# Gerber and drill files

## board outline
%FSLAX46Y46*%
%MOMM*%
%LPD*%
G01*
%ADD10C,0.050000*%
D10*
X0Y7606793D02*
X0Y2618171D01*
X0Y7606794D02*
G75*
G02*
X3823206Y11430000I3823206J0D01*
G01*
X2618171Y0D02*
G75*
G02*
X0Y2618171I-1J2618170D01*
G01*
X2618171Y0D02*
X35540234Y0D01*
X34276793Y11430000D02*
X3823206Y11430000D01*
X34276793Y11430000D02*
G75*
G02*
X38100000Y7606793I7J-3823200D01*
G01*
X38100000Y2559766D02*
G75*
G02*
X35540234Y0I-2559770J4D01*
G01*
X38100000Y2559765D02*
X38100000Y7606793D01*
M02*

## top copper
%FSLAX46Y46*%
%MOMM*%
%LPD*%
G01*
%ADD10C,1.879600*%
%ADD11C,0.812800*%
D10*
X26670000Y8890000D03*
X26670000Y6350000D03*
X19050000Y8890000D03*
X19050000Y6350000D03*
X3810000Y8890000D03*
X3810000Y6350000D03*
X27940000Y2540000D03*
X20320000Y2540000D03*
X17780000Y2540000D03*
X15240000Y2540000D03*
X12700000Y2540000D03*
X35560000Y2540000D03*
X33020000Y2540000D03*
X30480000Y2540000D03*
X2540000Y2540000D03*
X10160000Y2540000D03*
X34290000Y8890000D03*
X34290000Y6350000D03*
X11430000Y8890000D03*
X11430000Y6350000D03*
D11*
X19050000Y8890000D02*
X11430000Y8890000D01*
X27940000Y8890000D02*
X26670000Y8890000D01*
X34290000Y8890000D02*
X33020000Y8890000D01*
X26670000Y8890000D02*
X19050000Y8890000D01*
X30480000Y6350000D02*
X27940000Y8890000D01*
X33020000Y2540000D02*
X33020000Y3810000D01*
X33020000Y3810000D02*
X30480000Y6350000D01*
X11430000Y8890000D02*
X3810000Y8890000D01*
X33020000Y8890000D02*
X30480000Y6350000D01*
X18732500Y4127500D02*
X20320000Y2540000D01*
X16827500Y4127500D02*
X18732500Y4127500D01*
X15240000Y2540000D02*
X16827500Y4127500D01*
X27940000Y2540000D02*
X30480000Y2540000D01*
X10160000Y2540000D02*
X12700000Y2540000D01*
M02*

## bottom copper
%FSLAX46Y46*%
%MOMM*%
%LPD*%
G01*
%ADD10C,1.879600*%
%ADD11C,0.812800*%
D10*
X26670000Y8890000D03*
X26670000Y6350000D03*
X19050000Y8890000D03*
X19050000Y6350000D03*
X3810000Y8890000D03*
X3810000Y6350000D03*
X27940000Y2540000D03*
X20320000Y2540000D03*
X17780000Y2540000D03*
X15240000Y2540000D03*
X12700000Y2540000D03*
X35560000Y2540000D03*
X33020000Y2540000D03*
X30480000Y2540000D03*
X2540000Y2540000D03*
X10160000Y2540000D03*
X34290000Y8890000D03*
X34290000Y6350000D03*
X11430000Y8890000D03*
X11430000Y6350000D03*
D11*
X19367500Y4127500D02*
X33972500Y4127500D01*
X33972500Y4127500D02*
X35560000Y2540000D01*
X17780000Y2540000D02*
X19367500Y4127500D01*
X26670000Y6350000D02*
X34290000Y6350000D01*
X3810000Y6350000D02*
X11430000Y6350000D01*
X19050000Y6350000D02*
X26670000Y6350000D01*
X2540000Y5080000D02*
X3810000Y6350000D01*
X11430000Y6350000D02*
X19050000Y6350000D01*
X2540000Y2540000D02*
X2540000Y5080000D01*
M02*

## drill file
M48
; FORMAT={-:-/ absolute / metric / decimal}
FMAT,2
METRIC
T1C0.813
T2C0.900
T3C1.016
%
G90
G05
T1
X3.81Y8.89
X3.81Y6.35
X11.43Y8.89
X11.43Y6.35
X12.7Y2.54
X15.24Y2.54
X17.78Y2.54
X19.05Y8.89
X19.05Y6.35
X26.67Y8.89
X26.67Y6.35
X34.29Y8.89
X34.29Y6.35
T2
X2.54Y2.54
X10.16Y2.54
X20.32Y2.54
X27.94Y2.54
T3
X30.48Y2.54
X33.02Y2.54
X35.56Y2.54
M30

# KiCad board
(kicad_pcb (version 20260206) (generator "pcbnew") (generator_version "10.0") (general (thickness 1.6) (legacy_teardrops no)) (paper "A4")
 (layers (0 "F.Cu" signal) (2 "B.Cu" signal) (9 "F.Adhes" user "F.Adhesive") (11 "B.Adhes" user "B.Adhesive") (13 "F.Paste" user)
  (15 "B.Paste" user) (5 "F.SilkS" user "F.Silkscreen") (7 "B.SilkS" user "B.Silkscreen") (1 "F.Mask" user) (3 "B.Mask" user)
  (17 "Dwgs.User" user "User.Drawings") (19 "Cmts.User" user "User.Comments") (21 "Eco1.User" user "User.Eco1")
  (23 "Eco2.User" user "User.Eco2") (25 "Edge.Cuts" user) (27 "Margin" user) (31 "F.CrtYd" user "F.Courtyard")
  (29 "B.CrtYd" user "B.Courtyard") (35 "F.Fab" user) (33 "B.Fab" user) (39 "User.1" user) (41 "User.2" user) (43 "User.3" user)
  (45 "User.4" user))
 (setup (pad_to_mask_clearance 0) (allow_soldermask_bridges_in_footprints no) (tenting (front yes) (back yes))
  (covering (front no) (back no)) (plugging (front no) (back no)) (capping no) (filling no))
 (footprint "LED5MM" (layer "F.Cu") (at 26.67 -7.62 -90)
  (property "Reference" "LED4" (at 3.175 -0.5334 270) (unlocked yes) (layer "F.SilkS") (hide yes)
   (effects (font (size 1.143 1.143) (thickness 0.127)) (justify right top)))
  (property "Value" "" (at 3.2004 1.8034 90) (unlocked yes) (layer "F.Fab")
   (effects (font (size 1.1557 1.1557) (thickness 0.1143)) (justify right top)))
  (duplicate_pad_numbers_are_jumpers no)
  (pad "A" thru_hole circle (at -1.27 0 270) (size 1.8796 1.8796) (drill 0.8128) (layers "*.Cu" "*.Mask") (remove_unused_layers no)
   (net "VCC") (solder_mask_margin 0.1016) (thermal_bridge_angle 0))
  (pad "K" thru_hole circle (at 1.27 0 270) (size 1.8796 1.8796) (drill 0.8128) (layers "*.Cu" "*.Mask") (remove_unused_layers no)
   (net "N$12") (solder_mask_margin 0.1016) (thermal_bridge_angle 0)))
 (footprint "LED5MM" (layer "F.Cu") (at 19.05 -7.62 -90)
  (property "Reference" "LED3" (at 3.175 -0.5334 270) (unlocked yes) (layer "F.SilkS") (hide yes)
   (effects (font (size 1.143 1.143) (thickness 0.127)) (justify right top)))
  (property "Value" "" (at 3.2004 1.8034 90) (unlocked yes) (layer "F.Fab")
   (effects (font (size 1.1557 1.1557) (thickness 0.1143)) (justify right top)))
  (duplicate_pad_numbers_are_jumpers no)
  (pad "A" thru_hole circle (at -1.27 0 270) (size 1.8796 1.8796) (drill 0.8128) (layers "*.Cu" "*.Mask") (remove_unused_layers no)
   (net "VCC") (solder_mask_margin 0.1016) (thermal_bridge_angle 0))
  (pad "K" thru_hole circle (at 1.27 0 270) (size 1.8796 1.8796) (drill 0.8128) (layers "*.Cu" "*.Mask") (remove_unused_layers no)
   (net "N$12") (solder_mask_margin 0.1016) (thermal_bridge_angle 0)))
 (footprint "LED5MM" (layer "F.Cu") (at 3.81 -7.62 -90)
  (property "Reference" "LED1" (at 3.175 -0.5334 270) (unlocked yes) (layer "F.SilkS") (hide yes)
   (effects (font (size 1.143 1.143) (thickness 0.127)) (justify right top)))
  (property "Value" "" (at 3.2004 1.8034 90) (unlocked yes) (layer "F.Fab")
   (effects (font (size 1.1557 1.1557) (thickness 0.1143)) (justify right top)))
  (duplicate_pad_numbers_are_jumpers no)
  (pad "A" thru_hole circle (at -1.27 0 270) (size 1.8796 1.8796) (drill 0.8128) (layers "*.Cu" "*.Mask") (remove_unused_layers no)
   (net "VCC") (solder_mask_margin 0.1016) (thermal_bridge_angle 0))
  (pad "K" thru_hole circle (at 1.27 0 270) (size 1.8796 1.8796) (drill 0.8128) (layers "*.Cu" "*.Mask") (remove_unused_layers no)
   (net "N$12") (solder_mask_margin 0.1016) (thermal_bridge_angle 0)))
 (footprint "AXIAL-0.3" (layer "F.Cu") (at 24.13 -2.54 180)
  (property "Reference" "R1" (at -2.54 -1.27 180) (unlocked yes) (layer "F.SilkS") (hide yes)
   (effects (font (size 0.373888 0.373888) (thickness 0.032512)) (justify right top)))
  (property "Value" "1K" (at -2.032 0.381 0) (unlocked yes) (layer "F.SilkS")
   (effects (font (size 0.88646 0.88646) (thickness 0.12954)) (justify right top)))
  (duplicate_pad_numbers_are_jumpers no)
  (pad "P$1" thru_hole circle (at -3.81 0 180) (size 1.8796 1.8796) (drill 0.9) (layers "*.Cu" "*.Mask") (remove_unused_layers no)
   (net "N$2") (solder_mask_margin 0.1016) (thermal_bridge_angle 0))
  (pad "P$2" thru_hole circle (at 3.81 0 180) (size 1.8796 1.8796) (drill 0.9) (layers "*.Cu" "*.Mask") (remove_unused_layers no)
   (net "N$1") (solder_mask_margin 0.1016) (thermal_bridge_angle 0)))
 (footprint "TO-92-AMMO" (layer "F.Cu") (at 15.24 -2.54 180)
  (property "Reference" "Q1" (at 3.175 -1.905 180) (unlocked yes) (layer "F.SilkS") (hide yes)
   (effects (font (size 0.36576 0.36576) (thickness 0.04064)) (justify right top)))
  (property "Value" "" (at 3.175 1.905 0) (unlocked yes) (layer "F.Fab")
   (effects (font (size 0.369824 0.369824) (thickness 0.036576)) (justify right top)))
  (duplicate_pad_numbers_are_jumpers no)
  (pad "1" thru_hole circle (at -2.54 0 180) (size 1.8796 1.8796) (drill 0.8128) (layers "*.Cu" "*.Mask") (remove_unused_layers no)
   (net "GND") (solder_mask_margin 0.1016) (thermal_bridge_angle 0))
  (pad "2" thru_hole circle (at 0 0 180) (size 1.8796 1.8796) (drill 0.8128) (layers "*.Cu" "*.Mask") (remove_unused_layers no) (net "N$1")
   (solder_mask_margin 0.1016) (thermal_bridge_angle 0))
  (pad "3" thru_hole circle (at 2.54 0 180) (size 1.8796 1.8796) (drill 0.8128) (layers "*.Cu" "*.Mask") (remove_unused_layers no)
   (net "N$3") (solder_mask_margin 0.1016) (thermal_bridge_angle 0)))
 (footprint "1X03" (layer "F.Cu") (at 35.56 -2.54 180)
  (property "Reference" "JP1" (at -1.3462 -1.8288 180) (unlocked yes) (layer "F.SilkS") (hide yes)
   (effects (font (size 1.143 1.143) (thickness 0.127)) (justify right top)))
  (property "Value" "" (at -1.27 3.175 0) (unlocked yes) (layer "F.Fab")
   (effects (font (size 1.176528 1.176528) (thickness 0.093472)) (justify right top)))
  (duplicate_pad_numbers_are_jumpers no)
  (pad "1" thru_hole circle (at 0 0 270) (size 1.8796 1.8796) (drill 1.016) (layers "*.Cu" "*.Mask") (remove_unused_layers no) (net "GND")
   (solder_mask_margin 0.1016) (thermal_bridge_angle 0))
  (pad "2" thru_hole circle (at 2.54 0 270) (size 1.8796 1.8796) (drill 1.016) (layers "*.Cu" "*.Mask") (remove_unused_layers no)
   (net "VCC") (solder_mask_margin 0.1016) (thermal_bridge_angle 0))
  (pad "3" thru_hole circle (at 5.08 0 270) (size 1.8796 1.8796) (drill 1.016) (layers "*.Cu" "*.Mask") (remove_unused_layers no)
   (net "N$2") (solder_mask_margin 0.1016) (thermal_bridge_angle 0)))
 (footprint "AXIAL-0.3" (layer "F.Cu") (at 6.35 -2.54)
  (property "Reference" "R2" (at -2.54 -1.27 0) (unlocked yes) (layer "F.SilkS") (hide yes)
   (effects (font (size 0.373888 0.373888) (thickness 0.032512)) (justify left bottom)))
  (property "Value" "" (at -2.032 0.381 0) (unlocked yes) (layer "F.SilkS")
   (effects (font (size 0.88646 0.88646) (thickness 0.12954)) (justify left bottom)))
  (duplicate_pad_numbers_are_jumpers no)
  (pad "P$1" thru_hole circle (at -3.81 0) (size 1.8796 1.8796) (drill 0.9) (layers "*.Cu" "*.Mask") (remove_unused_layers no) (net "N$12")
   (solder_mask_margin 0.1016) (thermal_bridge_angle 0))
  (pad "P$2" thru_hole circle (at 3.81 0) (size 1.8796 1.8796) (drill 0.9) (layers "*.Cu" "*.Mask") (remove_unused_layers no) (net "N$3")
   (solder_mask_margin 0.1016) (thermal_bridge_angle 0)))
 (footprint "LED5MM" (layer "F.Cu") (at 34.29 -7.62 -90)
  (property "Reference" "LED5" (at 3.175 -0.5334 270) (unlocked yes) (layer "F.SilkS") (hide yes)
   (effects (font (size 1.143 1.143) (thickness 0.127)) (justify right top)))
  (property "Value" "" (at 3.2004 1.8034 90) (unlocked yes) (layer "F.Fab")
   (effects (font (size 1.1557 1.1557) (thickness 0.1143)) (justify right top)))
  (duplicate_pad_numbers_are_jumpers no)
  (pad "A" thru_hole circle (at -1.27 0 270) (size 1.8796 1.8796) (drill 0.8128) (layers "*.Cu" "*.Mask") (remove_unused_layers no)
   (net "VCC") (solder_mask_margin 0.1016) (thermal_bridge_angle 0))
  (pad "K" thru_hole circle (at 1.27 0 270) (size 1.8796 1.8796) (drill 0.8128) (layers "*.Cu" "*.Mask") (remove_unused_layers no)
   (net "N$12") (solder_mask_margin 0.1016) (thermal_bridge_angle 0)))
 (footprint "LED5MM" (layer "F.Cu") (at 11.43 -7.62 -90)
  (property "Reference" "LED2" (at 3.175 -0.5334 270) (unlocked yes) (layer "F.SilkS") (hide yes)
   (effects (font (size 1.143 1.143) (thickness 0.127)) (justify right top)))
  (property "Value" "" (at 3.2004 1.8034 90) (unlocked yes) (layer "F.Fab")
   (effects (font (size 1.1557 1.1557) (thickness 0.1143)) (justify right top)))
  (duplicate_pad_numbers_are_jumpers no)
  (pad "A" thru_hole circle (at -1.27 0 270) (size 1.8796 1.8796) (drill 0.8128) (layers "*.Cu" "*.Mask") (remove_unused_layers no)
   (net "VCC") (solder_mask_margin 0.1016) (thermal_bridge_angle 0))
  (pad "K" thru_hole circle (at 1.27 0 270) (size 1.8796 1.8796) (drill 0.8128) (layers "*.Cu" "*.Mask") (remove_unused_layers no)
   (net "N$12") (solder_mask_margin 0.1016) (thermal_bridge_angle 0)))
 (gr_line (start 0 -7.606793) (end 0 -2.618171) (stroke (width 0.05) (type solid)) (layer "Edge.Cuts"))
 (gr_arc (start 0 -7.606794) (mid 1.119791 -10.310209) (end 3.823206 -11.43) (stroke (width 0.05) (type solid)) (layer "Edge.Cuts"))
 (gr_arc (start 2.618171 0) (mid 0.766845 -0.766845) (end 0 -2.618171) (stroke (width 0.05) (type solid)) (layer "Edge.Cuts"))
 (gr_line (start 2.618171 0) (end 35.540234 0) (stroke (width 0.05) (type solid)) (layer "Edge.Cuts"))
 (gr_line (start 34.276793 -11.43) (end 3.823206 -11.43) (stroke (width 0.05) (type solid)) (layer "Edge.Cuts"))
 (gr_arc (start 34.276793 -11.43) (mid 36.980209 -10.310209) (end 38.1 -7.606793) (stroke (width 0.05) (type solid)) (layer "Edge.Cuts"))
 (gr_arc (start 38.1 -2.559766) (mid 37.350262 -0.749738) (end 35.540234 0) (stroke (width 0.05) (type solid)) (layer "Edge.Cuts"))
 (gr_line (start 38.1 -2.559765) (end 38.1 -7.606793) (stroke (width 0.05) (type solid)) (layer "Edge.Cuts"))
 (segment (start 19.3675 -4.1275) (end 33.9725 -4.1275) (width 0.8128) (layer "B.Cu") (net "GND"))
 (segment (start 33.9725 -4.1275) (end 35.56 -2.54) (width 0.8128) (layer "B.Cu") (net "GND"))
 (segment (start 17.78 -2.54) (end 19.3675 -4.1275) (width 0.8128) (layer "B.Cu") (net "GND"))
 (segment (start 19.05 -8.89) (end 11.43 -8.89) (width 0.8128) (layer "F.Cu") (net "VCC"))
 (segment (start 27.94 -8.89) (end 26.67 -8.89) (width 0.8128) (layer "F.Cu") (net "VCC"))
 (segment (start 34.29 -8.89) (end 33.02 -8.89) (width 0.8128) (layer "F.Cu") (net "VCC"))
 (segment (start 26.67 -8.89) (end 19.05 -8.89) (width 0.8128) (layer "F.Cu") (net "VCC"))
 (segment (start 30.48 -6.35) (end 27.94 -8.89) (width 0.8128) (layer "F.Cu") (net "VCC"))
 (segment (start 33.02 -2.54) (end 33.02 -3.81) (width 0.8128) (layer "F.Cu") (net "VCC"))
 (segment (start 33.02 -3.81) (end 30.48 -6.35) (width 0.8128) (layer "F.Cu") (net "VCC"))
 (segment (start 11.43 -8.89) (end 3.81 -8.89) (width 0.8128) (layer "F.Cu") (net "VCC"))
 (segment (start 33.02 -8.89) (end 30.48 -6.35) (width 0.8128) (layer "F.Cu") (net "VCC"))
 (segment (start 18.7325 -4.1275) (end 20.32 -2.54) (width 0.8128) (layer "F.Cu") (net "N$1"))
 (segment (start 16.8275 -4.1275) (end 18.7325 -4.1275) (width 0.8128) (layer "F.Cu") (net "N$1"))
 (segment (start 15.24 -2.54) (end 16.8275 -4.1275) (width 0.8128) (layer "F.Cu") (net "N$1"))
 (segment (start 27.94 -2.54) (end 30.48 -2.54) (width 0.8128) (layer "F.Cu") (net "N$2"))
 (segment (start 26.67 -6.35) (end 34.29 -6.35) (width 0.8128) (layer "B.Cu") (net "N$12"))
 (segment (start 3.81 -6.35) (end 11.43 -6.35) (width 0.8128) (layer "B.Cu") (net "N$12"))
 (segment (start 19.05 -6.35) (end 26.67 -6.35) (width 0.8128) (layer "B.Cu") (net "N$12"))
 (segment (start 2.54 -5.08) (end 3.81 -6.35) (width 0.8128) (layer "B.Cu") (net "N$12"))
 (segment (start 11.43 -6.35) (end 19.05 -6.35) (width 0.8128) (layer "B.Cu") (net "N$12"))
 (segment (start 2.54 -2.54) (end 2.54 -5.08) (width 0.8128) (layer "B.Cu") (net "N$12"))
 (segment (start 10.16 -2.54) (end 12.7 -2.54) (width 0.8128) (layer "F.Cu") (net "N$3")))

